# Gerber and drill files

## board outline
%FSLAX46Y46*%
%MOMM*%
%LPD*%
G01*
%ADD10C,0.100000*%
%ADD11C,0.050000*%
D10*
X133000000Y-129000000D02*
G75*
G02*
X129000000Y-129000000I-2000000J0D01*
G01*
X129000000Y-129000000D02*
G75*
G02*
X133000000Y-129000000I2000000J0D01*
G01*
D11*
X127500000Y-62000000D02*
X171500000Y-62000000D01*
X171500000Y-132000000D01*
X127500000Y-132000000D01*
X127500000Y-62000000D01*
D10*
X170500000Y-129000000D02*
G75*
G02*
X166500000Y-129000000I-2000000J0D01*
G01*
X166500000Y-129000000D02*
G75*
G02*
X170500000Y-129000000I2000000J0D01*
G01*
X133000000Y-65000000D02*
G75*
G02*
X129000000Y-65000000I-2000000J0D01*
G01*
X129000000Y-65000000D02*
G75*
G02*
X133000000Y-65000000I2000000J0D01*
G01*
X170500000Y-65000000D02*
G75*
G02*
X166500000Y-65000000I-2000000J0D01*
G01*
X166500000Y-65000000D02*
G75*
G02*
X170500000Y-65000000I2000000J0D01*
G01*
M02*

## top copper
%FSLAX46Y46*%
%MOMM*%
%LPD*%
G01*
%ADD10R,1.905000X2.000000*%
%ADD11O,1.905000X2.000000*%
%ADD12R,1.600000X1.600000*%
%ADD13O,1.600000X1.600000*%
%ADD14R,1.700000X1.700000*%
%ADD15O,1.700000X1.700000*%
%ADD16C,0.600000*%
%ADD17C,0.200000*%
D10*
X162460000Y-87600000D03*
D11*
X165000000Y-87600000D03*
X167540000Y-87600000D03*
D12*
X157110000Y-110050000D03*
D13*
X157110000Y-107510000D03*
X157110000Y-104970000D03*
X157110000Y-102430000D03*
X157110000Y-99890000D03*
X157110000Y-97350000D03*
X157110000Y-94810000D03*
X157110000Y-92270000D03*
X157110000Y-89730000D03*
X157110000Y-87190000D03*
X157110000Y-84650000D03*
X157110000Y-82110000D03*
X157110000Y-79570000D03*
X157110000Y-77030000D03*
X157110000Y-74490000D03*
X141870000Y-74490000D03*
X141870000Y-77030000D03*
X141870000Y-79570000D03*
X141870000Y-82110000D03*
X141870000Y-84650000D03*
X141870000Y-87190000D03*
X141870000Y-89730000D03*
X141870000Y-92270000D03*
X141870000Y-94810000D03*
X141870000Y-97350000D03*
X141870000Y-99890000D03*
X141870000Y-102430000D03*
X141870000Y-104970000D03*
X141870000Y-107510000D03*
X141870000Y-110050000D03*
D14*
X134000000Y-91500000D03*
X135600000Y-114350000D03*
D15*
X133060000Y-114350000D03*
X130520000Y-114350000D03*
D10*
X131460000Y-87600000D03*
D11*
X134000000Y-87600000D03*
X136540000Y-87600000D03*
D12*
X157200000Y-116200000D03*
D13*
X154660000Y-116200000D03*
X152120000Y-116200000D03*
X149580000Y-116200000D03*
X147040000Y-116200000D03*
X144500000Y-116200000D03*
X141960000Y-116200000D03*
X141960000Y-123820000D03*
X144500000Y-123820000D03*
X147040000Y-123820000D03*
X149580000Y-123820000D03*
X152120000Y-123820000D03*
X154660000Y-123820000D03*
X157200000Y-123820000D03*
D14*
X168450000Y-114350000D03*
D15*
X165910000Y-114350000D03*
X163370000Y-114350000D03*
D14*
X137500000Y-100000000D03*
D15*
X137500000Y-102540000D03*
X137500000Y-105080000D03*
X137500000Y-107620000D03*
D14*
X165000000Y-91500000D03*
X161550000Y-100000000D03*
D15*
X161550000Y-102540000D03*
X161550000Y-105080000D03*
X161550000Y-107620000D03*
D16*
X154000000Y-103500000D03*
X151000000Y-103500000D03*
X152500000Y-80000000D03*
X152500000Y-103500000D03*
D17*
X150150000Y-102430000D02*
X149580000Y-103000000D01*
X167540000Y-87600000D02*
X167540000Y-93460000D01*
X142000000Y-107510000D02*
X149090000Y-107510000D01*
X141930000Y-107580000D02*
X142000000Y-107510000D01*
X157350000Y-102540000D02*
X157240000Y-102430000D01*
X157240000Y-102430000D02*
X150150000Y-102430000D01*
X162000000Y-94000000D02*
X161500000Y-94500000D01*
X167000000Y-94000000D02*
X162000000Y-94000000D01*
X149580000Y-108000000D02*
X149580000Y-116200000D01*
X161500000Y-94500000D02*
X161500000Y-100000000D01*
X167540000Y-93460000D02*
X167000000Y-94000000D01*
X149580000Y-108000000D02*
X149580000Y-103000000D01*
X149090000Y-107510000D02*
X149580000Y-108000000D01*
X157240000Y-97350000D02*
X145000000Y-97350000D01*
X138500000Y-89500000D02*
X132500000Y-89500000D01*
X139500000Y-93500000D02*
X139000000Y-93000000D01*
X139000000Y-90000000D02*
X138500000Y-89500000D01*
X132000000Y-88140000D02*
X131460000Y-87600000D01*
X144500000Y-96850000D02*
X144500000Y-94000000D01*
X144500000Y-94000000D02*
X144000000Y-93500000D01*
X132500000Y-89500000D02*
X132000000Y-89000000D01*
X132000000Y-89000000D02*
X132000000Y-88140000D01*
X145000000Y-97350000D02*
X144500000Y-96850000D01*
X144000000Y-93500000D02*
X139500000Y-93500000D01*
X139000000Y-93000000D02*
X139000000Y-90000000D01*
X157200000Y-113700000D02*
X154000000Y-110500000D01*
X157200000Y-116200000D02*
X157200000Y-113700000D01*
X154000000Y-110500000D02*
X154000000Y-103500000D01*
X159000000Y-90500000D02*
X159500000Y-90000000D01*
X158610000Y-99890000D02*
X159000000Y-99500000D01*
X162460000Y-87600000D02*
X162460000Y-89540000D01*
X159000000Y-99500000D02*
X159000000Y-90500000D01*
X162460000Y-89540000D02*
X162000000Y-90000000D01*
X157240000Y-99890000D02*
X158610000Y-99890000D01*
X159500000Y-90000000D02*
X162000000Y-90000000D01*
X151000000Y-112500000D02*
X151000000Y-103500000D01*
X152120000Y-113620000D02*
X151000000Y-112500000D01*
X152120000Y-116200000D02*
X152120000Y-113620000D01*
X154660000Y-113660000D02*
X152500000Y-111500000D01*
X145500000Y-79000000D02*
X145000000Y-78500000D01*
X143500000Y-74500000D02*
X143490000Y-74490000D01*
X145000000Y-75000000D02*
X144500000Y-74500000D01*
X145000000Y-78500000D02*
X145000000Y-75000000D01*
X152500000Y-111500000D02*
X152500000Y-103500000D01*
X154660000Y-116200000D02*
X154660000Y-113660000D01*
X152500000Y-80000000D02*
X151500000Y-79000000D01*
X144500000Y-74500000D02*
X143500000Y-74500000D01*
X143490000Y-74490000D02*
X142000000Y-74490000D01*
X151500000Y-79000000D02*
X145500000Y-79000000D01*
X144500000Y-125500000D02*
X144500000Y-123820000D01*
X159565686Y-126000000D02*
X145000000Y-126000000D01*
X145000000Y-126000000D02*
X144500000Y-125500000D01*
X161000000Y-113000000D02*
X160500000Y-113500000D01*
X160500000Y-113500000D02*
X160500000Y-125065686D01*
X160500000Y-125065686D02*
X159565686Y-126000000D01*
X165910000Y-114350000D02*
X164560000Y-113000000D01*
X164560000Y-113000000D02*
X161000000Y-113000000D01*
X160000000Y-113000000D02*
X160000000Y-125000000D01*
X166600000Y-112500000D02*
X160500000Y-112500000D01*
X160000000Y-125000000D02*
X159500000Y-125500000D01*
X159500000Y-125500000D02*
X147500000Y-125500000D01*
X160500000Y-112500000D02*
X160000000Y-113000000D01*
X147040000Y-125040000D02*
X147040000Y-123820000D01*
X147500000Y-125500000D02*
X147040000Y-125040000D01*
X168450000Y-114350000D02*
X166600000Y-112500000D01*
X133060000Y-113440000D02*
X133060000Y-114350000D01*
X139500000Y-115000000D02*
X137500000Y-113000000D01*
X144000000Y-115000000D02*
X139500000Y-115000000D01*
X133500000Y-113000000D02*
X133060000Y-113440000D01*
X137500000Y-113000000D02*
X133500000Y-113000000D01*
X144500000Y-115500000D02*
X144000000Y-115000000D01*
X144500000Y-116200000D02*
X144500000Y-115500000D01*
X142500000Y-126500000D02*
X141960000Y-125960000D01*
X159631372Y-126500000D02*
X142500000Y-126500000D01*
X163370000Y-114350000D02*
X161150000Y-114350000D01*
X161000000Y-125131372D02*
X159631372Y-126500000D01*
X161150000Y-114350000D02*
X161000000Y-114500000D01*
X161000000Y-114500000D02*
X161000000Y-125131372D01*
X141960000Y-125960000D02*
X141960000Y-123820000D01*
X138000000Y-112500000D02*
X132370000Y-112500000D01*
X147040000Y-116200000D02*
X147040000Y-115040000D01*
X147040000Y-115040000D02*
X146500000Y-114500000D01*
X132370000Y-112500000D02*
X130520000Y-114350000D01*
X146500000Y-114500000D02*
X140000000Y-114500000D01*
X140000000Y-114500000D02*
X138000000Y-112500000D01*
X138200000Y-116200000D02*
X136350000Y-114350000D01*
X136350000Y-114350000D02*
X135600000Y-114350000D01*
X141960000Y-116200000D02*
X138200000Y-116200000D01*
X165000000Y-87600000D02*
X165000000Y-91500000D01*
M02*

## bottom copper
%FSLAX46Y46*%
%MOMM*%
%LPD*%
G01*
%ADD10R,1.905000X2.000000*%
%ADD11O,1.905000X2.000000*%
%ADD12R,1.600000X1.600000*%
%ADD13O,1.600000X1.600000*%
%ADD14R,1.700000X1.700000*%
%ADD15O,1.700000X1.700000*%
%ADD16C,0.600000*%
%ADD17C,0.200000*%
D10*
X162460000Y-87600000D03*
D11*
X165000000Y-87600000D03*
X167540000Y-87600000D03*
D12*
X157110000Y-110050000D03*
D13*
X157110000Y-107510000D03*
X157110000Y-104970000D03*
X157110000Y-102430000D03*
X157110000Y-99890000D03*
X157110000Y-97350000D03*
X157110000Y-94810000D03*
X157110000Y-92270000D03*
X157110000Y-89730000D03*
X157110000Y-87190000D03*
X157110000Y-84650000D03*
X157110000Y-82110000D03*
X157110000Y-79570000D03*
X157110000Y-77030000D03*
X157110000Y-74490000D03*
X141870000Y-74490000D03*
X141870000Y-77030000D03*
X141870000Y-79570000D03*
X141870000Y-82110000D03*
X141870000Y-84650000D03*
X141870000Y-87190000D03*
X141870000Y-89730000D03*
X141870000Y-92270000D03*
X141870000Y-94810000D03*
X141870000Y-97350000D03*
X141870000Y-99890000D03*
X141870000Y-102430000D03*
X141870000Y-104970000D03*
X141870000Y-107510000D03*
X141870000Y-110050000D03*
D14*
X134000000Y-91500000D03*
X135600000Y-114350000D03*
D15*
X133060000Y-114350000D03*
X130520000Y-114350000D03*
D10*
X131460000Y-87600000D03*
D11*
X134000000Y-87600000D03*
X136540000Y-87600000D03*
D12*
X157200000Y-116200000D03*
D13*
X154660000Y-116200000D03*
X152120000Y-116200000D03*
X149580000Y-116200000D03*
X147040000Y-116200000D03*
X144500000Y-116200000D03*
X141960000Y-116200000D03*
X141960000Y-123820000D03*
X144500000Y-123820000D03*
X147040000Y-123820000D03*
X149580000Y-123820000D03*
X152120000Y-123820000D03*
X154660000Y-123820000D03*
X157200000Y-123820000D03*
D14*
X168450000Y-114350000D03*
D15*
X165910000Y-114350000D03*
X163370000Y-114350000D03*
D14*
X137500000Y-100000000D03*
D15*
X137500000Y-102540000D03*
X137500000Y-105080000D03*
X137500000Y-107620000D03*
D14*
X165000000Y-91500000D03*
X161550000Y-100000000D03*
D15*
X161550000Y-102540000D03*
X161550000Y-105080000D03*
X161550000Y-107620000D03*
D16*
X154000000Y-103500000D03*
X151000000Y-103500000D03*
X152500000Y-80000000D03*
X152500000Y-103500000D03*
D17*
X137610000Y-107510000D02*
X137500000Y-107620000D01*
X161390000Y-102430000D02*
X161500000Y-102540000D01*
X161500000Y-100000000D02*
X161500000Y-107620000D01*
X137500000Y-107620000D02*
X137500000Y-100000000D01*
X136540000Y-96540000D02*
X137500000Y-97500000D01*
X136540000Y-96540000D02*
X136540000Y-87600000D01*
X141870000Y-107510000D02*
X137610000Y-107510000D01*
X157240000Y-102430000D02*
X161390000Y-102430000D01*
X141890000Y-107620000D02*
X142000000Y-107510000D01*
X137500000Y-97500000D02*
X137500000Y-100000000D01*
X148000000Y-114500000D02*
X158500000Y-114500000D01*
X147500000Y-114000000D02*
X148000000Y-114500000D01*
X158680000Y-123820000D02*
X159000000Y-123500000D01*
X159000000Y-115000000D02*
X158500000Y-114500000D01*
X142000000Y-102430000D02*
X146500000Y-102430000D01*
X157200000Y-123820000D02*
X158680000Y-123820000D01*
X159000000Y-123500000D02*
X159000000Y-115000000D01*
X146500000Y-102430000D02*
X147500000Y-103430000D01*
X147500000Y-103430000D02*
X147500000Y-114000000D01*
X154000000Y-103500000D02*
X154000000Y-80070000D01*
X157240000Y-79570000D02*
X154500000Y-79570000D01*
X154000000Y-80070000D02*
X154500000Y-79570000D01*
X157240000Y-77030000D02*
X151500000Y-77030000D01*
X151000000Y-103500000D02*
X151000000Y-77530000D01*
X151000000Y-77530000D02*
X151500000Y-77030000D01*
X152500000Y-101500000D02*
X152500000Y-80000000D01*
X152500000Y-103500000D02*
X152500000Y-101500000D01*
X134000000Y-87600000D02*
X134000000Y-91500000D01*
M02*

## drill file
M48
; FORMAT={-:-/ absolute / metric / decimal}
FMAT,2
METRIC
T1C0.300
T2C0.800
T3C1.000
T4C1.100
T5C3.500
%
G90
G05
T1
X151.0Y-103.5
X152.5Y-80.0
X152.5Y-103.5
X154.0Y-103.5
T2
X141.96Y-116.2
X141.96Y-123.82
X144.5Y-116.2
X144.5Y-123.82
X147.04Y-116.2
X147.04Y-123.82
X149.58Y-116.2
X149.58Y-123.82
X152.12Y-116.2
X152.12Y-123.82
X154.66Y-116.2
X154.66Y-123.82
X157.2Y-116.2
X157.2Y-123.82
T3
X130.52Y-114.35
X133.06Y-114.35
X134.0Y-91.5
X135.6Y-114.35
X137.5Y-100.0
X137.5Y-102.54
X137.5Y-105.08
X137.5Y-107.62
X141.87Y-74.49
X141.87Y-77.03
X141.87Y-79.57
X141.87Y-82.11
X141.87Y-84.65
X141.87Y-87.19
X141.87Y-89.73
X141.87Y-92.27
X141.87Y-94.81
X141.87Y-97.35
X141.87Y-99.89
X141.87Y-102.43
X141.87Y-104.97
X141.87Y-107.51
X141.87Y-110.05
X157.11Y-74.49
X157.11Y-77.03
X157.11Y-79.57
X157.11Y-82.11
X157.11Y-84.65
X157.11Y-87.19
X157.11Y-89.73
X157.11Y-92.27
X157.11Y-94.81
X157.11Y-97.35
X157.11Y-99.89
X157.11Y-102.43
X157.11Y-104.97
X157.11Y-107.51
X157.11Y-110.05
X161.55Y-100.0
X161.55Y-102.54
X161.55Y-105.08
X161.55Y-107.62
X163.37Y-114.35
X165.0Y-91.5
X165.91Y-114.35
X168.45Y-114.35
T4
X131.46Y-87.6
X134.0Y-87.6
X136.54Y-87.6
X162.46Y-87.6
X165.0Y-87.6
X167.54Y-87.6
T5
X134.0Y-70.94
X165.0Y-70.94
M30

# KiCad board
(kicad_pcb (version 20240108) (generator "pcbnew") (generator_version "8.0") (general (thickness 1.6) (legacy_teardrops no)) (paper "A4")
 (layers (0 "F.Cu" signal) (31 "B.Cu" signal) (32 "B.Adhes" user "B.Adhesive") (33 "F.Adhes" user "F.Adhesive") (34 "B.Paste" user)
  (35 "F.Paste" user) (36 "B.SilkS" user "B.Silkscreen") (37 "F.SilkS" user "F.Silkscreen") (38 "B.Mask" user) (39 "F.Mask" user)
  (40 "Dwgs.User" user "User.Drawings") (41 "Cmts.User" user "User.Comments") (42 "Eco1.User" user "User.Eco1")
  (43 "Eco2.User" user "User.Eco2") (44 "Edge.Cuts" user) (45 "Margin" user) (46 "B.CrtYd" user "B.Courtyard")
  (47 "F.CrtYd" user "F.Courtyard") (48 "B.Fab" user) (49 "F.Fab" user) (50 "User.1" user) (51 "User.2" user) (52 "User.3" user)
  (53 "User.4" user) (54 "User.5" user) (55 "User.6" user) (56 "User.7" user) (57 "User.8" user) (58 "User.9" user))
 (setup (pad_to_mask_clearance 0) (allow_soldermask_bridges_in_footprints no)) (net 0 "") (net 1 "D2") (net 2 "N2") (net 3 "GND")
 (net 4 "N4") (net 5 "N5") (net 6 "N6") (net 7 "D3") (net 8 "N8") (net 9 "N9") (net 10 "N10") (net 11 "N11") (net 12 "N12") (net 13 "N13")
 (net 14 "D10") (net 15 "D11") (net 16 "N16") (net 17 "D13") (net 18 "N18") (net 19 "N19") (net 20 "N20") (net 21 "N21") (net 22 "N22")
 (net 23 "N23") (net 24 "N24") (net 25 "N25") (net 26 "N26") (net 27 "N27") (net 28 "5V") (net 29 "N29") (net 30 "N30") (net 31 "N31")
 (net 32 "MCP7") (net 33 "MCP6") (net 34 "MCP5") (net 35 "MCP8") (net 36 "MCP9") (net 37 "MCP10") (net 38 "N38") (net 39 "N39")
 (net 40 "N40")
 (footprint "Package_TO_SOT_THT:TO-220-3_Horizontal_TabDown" (layer "F.Cu") (at 162.46 87.6)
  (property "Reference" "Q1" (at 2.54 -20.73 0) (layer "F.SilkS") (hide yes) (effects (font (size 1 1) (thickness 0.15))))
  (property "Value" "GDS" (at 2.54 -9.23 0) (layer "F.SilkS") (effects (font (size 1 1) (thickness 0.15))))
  (pad "" np_thru_hole oval (at 2.54 -16.66) (size 3.5 3.5) (drill 3.5) (layers "*.Cu" "*.Mask"))
  (pad "1" thru_hole rect (at 0 0) (size 1.905 2) (drill 1.1) (layers "*.Cu" "*.Mask") (remove_unused_layers no) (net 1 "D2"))
  (pad "2" thru_hole oval (at 2.54 0) (size 1.905 2) (drill 1.1) (layers "*.Cu" "*.Mask") (remove_unused_layers no) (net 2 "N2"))
  (pad "3" thru_hole oval (at 5.08 0) (size 1.905 2) (drill 1.1) (layers "*.Cu" "*.Mask") (remove_unused_layers no) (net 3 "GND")))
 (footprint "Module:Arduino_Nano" (layer "F.Cu") (at 157.11 110.05 180)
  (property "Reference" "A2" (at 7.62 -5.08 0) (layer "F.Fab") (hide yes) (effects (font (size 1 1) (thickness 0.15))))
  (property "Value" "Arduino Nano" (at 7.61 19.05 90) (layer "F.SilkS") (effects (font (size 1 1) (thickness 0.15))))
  (pad "1" thru_hole rect (at 0 0 180) (size 1.6 1.6) (drill 1) (layers "*.Cu" "*.Mask") (remove_unused_layers no) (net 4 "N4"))
  (pad "2" thru_hole oval (at 0 2.54 180) (size 1.6 1.6) (drill 1) (layers "*.Cu" "*.Mask") (remove_unused_layers no) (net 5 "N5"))
  (pad "3" thru_hole oval (at 0 5.08 180) (size 1.6 1.6) (drill 1) (layers "*.Cu" "*.Mask") (remove_unused_layers no) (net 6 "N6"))
  (pad "4" thru_hole oval (at 0 7.62 180) (size 1.6 1.6) (drill 1) (layers "*.Cu" "*.Mask") (remove_unused_layers no) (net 3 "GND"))
  (pad "5" thru_hole oval (at 0 10.16 180) (size 1.6 1.6) (drill 1) (layers "*.Cu" "*.Mask") (remove_unused_layers no) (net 1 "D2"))
  (pad "6" thru_hole oval (at 0 12.7 180) (size 1.6 1.6) (drill 1) (layers "*.Cu" "*.Mask") (remove_unused_layers no) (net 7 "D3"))
  (pad "7" thru_hole oval (at 0 15.24 180) (size 1.6 1.6) (drill 1) (layers "*.Cu" "*.Mask") (remove_unused_layers no) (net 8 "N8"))
  (pad "8" thru_hole oval (at 0 17.78 180) (size 1.6 1.6) (drill 1) (layers "*.Cu" "*.Mask") (remove_unused_layers no) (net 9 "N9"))
  (pad "9" thru_hole oval (at 0 20.32 180) (size 1.6 1.6) (drill 1) (layers "*.Cu" "*.Mask") (remove_unused_layers no) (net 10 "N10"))
  (pad "10" thru_hole oval (at 0 22.86 180) (size 1.6 1.6) (drill 1) (layers "*.Cu" "*.Mask") (remove_unused_layers no) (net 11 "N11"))
  (pad "11" thru_hole oval (at 0 25.4 180) (size 1.6 1.6) (drill 1) (layers "*.Cu" "*.Mask") (remove_unused_layers no) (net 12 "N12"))
  (pad "12" thru_hole oval (at 0 27.94 180) (size 1.6 1.6) (drill 1) (layers "*.Cu" "*.Mask") (remove_unused_layers no) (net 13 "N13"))
  (pad "13" thru_hole oval (at 0 30.48 180) (size 1.6 1.6) (drill 1) (layers "*.Cu" "*.Mask") (remove_unused_layers no) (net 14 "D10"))
  (pad "14" thru_hole oval (at 0 33.02 180) (size 1.6 1.6) (drill 1) (layers "*.Cu" "*.Mask") (remove_unused_layers no) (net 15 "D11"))
  (pad "15" thru_hole oval (at 0 35.56 180) (size 1.6 1.6) (drill 1) (layers "*.Cu" "*.Mask") (remove_unused_layers no) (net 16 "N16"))
  (pad "16" thru_hole oval (at 15.24 35.56 180) (size 1.6 1.6) (drill 1) (layers "*.Cu" "*.Mask") (remove_unused_layers no) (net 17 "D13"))
  (pad "17" thru_hole oval (at 15.24 33.02 180) (size 1.6 1.6) (drill 1) (layers "*.Cu" "*.Mask") (remove_unused_layers no) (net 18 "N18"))
  (pad "18" thru_hole oval (at 15.24 30.48 180) (size 1.6 1.6) (drill 1) (layers "*.Cu" "*.Mask") (remove_unused_layers no) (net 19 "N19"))
  (pad "19" thru_hole oval (at 15.24 27.94 180) (size 1.6 1.6) (drill 1) (layers "*.Cu" "*.Mask") (remove_unused_layers no) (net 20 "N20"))
  (pad "20" thru_hole oval (at 15.24 25.4 180) (size 1.6 1.6) (drill 1) (layers "*.Cu" "*.Mask") (remove_unused_layers no) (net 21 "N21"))
  (pad "21" thru_hole oval (at 15.24 22.86 180) (size 1.6 1.6) (drill 1) (layers "*.Cu" "*.Mask") (remove_unused_layers no) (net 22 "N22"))
  (pad "22" thru_hole oval (at 15.24 20.32 180) (size 1.6 1.6) (drill 1) (layers "*.Cu" "*.Mask") (remove_unused_layers no) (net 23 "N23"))
  (pad "23" thru_hole oval (at 15.24 17.78 180) (size 1.6 1.6) (drill 1) (layers "*.Cu" "*.Mask") (remove_unused_layers no) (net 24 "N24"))
  (pad "24" thru_hole oval (at 15.24 15.24 180) (size 1.6 1.6) (drill 1) (layers "*.Cu" "*.Mask") (remove_unused_layers no) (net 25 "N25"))
  (pad "25" thru_hole oval (at 15.24 12.7 180) (size 1.6 1.6) (drill 1) (layers "*.Cu" "*.Mask") (remove_unused_layers no) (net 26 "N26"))
  (pad "26" thru_hole oval (at 15.24 10.16 180) (size 1.6 1.6) (drill 1) (layers "*.Cu" "*.Mask") (remove_unused_layers no) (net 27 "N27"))
  (pad "27" thru_hole oval (at 15.24 7.62 180) (size 1.6 1.6) (drill 1) (layers "*.Cu" "*.Mask") (remove_unused_layers no) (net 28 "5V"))
  (pad "28" thru_hole oval (at 15.24 5.08 180) (size 1.6 1.6) (drill 1) (layers "*.Cu" "*.Mask") (remove_unused_layers no) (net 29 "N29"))
  (pad "29" thru_hole oval (at 15.24 2.54 180) (size 1.6 1.6) (drill 1) (layers "*.Cu" "*.Mask") (remove_unused_layers no) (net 3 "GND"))
  (pad "30" thru_hole oval (at 15.24 0 180) (size 1.6 1.6) (drill 1) (layers "*.Cu" "*.Mask") (remove_unused_layers no) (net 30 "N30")))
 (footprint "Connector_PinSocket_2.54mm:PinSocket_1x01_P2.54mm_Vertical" (layer "F.Cu") (at 134 91.5)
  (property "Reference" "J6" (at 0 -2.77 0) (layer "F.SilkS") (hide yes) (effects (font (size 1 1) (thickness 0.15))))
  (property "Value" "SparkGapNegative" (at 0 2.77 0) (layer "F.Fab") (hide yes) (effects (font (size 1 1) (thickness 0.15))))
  (pad "1" thru_hole rect (at 0 0) (size 1.7 1.7) (drill 1) (layers "*.Cu" "*.Mask") (remove_unused_layers no) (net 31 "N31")))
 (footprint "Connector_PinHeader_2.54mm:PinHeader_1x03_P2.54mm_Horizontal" (layer "F.Cu") (at 135.6 114.35 -90)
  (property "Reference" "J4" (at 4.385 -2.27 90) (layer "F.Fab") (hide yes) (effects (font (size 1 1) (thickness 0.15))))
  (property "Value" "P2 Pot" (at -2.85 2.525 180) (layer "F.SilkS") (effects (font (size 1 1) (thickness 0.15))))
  (pad "1" thru_hole rect (at 0 0 270) (size 1.7 1.7) (drill 1) (layers "*.Cu" "*.Mask") (remove_unused_layers no) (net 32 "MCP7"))
  (pad "2" thru_hole oval (at 0 2.54 270) (size 1.7 1.7) (drill 1) (layers "*.Cu" "*.Mask") (remove_unused_layers no) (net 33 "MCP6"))
  (pad "3" thru_hole oval (at 0 5.08 270) (size 1.7 1.7) (drill 1) (layers "*.Cu" "*.Mask") (remove_unused_layers no) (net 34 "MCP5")))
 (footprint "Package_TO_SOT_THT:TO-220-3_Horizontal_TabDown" (layer "F.Cu") (at 131.46 87.6)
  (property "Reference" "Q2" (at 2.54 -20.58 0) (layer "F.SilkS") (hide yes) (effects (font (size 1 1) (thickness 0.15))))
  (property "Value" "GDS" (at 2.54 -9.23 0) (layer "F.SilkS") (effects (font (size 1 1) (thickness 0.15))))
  (pad "" np_thru_hole oval (at 2.54 -16.66) (size 3.5 3.5) (drill 3.5) (layers "*.Cu" "*.Mask"))
  (pad "1" thru_hole rect (at 0 0) (size 1.905 2) (drill 1.1) (layers "*.Cu" "*.Mask") (remove_unused_layers no) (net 7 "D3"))
  (pad "2" thru_hole oval (at 2.54 0) (size 1.905 2) (drill 1.1) (layers "*.Cu" "*.Mask") (remove_unused_layers no) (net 31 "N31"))
  (pad "3" thru_hole oval (at 5.08 0) (size 1.905 2) (drill 1.1) (layers "*.Cu" "*.Mask") (remove_unused_layers no) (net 3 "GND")))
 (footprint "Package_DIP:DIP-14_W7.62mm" (layer "F.Cu") (at 157.2 116.2 -90)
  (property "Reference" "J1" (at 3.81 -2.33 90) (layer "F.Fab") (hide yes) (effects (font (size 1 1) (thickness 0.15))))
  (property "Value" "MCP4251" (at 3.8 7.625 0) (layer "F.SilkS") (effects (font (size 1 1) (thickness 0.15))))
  (pad "1" thru_hole rect (at 0 0 270) (size 1.6 1.6) (drill 0.8) (layers "*.Cu" "*.Mask") (remove_unused_layers no) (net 14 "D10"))
  (pad "2" thru_hole oval (at 0 2.54 270) (size 1.6 1.6) (drill 0.8) (layers "*.Cu" "*.Mask") (remove_unused_layers no) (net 17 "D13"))
  (pad "3" thru_hole oval (at 0 5.08 270) (size 1.6 1.6) (drill 0.8) (layers "*.Cu" "*.Mask") (remove_unused_layers no) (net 15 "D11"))
  (pad "4" thru_hole oval (at 0 7.62 270) (size 1.6 1.6) (drill 0.8) (layers "*.Cu" "*.Mask") (remove_unused_layers no) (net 3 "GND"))
  (pad "5" thru_hole oval (at 0 10.16 270) (size 1.6 1.6) (drill 0.8) (layers "*.Cu" "*.Mask") (remove_unused_layers no) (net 34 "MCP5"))
  (pad "6" thru_hole oval (at 0 12.7 270) (size 1.6 1.6) (drill 0.8) (layers "*.Cu" "*.Mask") (remove_unused_layers no) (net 33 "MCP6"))
  (pad "7" thru_hole oval (at 0 15.24 270) (size 1.6 1.6) (drill 0.8) (layers "*.Cu" "*.Mask") (remove_unused_layers no) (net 32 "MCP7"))
  (pad "8" thru_hole oval (at 7.62 15.24 270) (size 1.6 1.6) (drill 0.8) (layers "*.Cu" "*.Mask") (remove_unused_layers no) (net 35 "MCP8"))
  (pad "9" thru_hole oval (at 7.62 12.7 270) (size 1.6 1.6) (drill 0.8) (layers "*.Cu" "*.Mask") (remove_unused_layers no) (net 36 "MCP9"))
  (pad "10" thru_hole oval (at 7.62 10.16 270) (size 1.6 1.6) (drill 0.8) (layers "*.Cu" "*.Mask") (remove_unused_layers no)
   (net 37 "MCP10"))
  (pad "11" thru_hole oval (at 7.62 7.62 270) (size 1.6 1.6) (drill 0.8) (layers "*.Cu" "*.Mask") (remove_unused_layers no) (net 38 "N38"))
  (pad "12" thru_hole oval (at 7.62 5.08 270) (size 1.6 1.6) (drill 0.8) (layers "*.Cu" "*.Mask") (remove_unused_layers no) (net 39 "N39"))
  (pad "13" thru_hole oval (at 7.62 2.54 270) (size 1.6 1.6) (drill 0.8) (layers "*.Cu" "*.Mask") (remove_unused_layers no) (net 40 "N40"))
  (pad "14" thru_hole oval (at 7.62 0 270) (size 1.6 1.6) (drill 0.8) (layers "*.Cu" "*.Mask") (remove_unused_layers no) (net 28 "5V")))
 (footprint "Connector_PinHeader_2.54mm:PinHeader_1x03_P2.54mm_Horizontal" (layer "F.Cu") (at 168.45 114.35 -90)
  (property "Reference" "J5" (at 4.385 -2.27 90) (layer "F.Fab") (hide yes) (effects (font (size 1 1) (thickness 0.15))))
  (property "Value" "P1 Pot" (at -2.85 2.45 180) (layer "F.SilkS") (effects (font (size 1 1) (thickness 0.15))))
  (pad "1" thru_hole rect (at 0 0 270) (size 1.7 1.7) (drill 1) (layers "*.Cu" "*.Mask") (remove_unused_layers no) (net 37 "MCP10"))
  (pad "2" thru_hole oval (at 0 2.54 270) (size 1.7 1.7) (drill 1) (layers "*.Cu" "*.Mask") (remove_unused_layers no) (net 36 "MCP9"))
  (pad "3" thru_hole oval (at 0 5.08 270) (size 1.7 1.7) (drill 1) (layers "*.Cu" "*.Mask") (remove_unused_layers no) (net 35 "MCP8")))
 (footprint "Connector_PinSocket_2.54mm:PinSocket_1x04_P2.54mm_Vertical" (layer "F.Cu") (at 137.5 100)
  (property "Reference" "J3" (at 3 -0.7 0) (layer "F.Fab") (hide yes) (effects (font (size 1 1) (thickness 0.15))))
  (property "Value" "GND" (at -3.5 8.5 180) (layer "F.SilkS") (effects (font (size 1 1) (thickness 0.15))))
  (pad "1" thru_hole rect (at 0 0) (size 1.7 1.7) (drill 1) (layers "*.Cu" "*.Mask") (remove_unused_layers no) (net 3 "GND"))
  (pad "2" thru_hole oval (at 0 2.54) (size 1.7 1.7) (drill 1) (layers "*.Cu" "*.Mask") (remove_unused_layers no) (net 3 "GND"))
  (pad "3" thru_hole oval (at 0 5.08) (size 1.7 1.7) (drill 1) (layers "*.Cu" "*.Mask") (remove_unused_layers no) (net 3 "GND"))
  (pad "4" thru_hole oval (at 0 7.62) (size 1.7 1.7) (drill 1) (layers "*.Cu" "*.Mask") (remove_unused_layers no) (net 3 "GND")))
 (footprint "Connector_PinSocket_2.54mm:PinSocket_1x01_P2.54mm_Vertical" (layer "F.Cu") (at 165 91.5)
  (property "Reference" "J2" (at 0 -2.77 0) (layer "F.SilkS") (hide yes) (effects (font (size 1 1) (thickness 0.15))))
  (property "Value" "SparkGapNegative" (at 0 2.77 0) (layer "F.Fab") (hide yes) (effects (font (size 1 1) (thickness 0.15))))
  (pad "1" thru_hole rect (at 0 0) (size 1.7 1.7) (drill 1) (layers "*.Cu" "*.Mask") (remove_unused_layers no) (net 2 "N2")))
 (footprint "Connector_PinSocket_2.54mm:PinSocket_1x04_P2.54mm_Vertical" (layer "F.Cu") (at 161.55 100)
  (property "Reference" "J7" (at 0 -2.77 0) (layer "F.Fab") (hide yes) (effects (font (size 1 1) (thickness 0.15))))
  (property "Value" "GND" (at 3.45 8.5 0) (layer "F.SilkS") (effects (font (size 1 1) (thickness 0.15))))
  (pad "1" thru_hole rect (at 0 0) (size 1.7 1.7) (drill 1) (layers "*.Cu" "*.Mask") (remove_unused_layers no) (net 3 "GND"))
  (pad "2" thru_hole oval (at 0 2.54) (size 1.7 1.7) (drill 1) (layers "*.Cu" "*.Mask") (remove_unused_layers no) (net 3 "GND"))
  (pad "3" thru_hole oval (at 0 5.08) (size 1.7 1.7) (drill 1) (layers "*.Cu" "*.Mask") (remove_unused_layers no) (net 3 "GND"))
  (pad "4" thru_hole oval (at 0 7.62) (size 1.7 1.7) (drill 1) (layers "*.Cu" "*.Mask") (remove_unused_layers no) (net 3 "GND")))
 (gr_circle (center 131 129) (end 133 129) (stroke (width 0.1) (type default)) (fill none) (layer "Edge.Cuts"))
 (gr_rect (start 127.5 62) (end 171.5 132) (stroke (width 0.05) (type default)) (fill none) (layer "Edge.Cuts"))
 (gr_circle (center 168.5 129) (end 170.5 129) (stroke (width 0.1) (type default)) (fill none) (layer "Edge.Cuts"))
 (gr_circle (center 131 65) (end 133 65) (stroke (width 0.1) (type default)) (fill none) (layer "Edge.Cuts"))
 (gr_circle (center 168.5 65) (end 170.5 65) (stroke (width 0.1) (type default)) (fill none) (layer "Edge.Cuts"))
 (segment (start 150.15 102.43) (end 149.58 103) (width 0.2) (layer "F.Cu") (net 3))
 (segment (start 167.54 87.6) (end 167.54 93.46) (width 0.2) (layer "F.Cu") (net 3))
 (segment (start 142 107.51) (end 149.09 107.51) (width 0.2) (layer "F.Cu") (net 3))
 (segment (start 141.93 107.58) (end 142 107.51) (width 0.2) (layer "F.Cu") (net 3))
 (segment (start 157.35 102.54) (end 157.24 102.43) (width 0.2) (layer "F.Cu") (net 3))
 (segment (start 157.24 102.43) (end 150.15 102.43) (width 0.2) (layer "F.Cu") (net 3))
 (segment (start 162 94) (end 161.5 94.5) (width 0.2) (layer "F.Cu") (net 3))
 (segment (start 167 94) (end 162 94) (width 0.2) (layer "F.Cu") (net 3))
 (segment (start 149.58 108) (end 149.58 116.2) (width 0.2) (layer "F.Cu") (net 3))
 (segment (start 161.5 94.5) (end 161.5 100) (width 0.2) (layer "F.Cu") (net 3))
 (segment (start 167.54 93.46) (end 167 94) (width 0.2) (layer "F.Cu") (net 3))
 (segment (start 149.58 108) (end 149.58 103) (width 0.2) (layer "F.Cu") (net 3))
 (segment (start 149.09 107.51) (end 149.58 108) (width 0.2) (layer "F.Cu") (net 3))
 (segment (start 137.61 107.51) (end 137.5 107.62) (width 0.2) (layer "B.Cu") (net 3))
 (segment (start 161.39 102.43) (end 161.5 102.54) (width 0.2) (layer "B.Cu") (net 3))
 (segment (start 161.5 100) (end 161.5 107.62) (width 0.2) (layer "B.Cu") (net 3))
 (segment (start 137.5 107.62) (end 137.5 100) (width 0.2) (layer "B.Cu") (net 3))
 (segment (start 136.54 96.54) (end 137.5 97.5) (width 0.2) (layer "B.Cu") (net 3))
 (segment (start 136.54 96.54) (end 136.54 87.6) (width 0.2) (layer "B.Cu") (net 3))
 (segment (start 141.87 107.51) (end 137.61 107.51) (width 0.2) (layer "B.Cu") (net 3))
 (segment (start 157.24 102.43) (end 161.39 102.43) (width 0.2) (layer "B.Cu") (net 3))
 (segment (start 141.89 107.62) (end 142 107.51) (width 0.2) (layer "B.Cu") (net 3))
 (segment (start 137.5 97.5) (end 137.5 100) (width 0.2) (layer "B.Cu") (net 3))
 (segment (start 157.24 97.35) (end 145 97.35) (width 0.2) (layer "F.Cu") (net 7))
 (segment (start 138.5 89.5) (end 132.5 89.5) (width 0.2) (layer "F.Cu") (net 7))
 (segment (start 139.5 93.5) (end 139 93) (width 0.2) (layer "F.Cu") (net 7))
 (segment (start 139 90) (end 138.5 89.5) (width 0.2) (layer "F.Cu") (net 7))
 (segment (start 132 88.14) (end 131.46 87.6) (width 0.2) (layer "F.Cu") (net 7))
 (segment (start 144.5 96.85) (end 144.5 94) (width 0.2) (layer "F.Cu") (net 7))
 (segment (start 144.5 94) (end 144 93.5) (width 0.2) (layer "F.Cu") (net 7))
 (segment (start 132.5 89.5) (end 132 89) (width 0.2) (layer "F.Cu") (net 7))
 (segment (start 132 89) (end 132 88.14) (width 0.2) (layer "F.Cu") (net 7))
 (segment (start 145 97.35) (end 144.5 96.85) (width 0.2) (layer "F.Cu") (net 7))
 (segment (start 144 93.5) (end 139.5 93.5) (width 0.2) (layer "F.Cu") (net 7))
 (segment (start 139 93) (end 139 90) (width 0.2) (layer "F.Cu") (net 7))
 (segment (start 148 114.5) (end 158.5 114.5) (width 0.2) (layer "B.Cu") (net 28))
 (segment (start 147.5 114) (end 148 114.5) (width 0.2) (layer "B.Cu") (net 28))
 (segment (start 158.68 123.82) (end 159 123.5) (width 0.2) (layer "B.Cu") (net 28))
 (segment (start 159 115) (end 158.5 114.5) (width 0.2) (layer "B.Cu") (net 28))
 (segment (start 142 102.43) (end 146.5 102.43) (width 0.2) (layer "B.Cu") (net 28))
 (segment (start 157.2 123.82) (end 158.68 123.82) (width 0.2) (layer "B.Cu") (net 28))
 (segment (start 159 123.5) (end 159 115) (width 0.2) (layer "B.Cu") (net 28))
 (segment (start 146.5 102.43) (end 147.5 103.43) (width 0.2) (layer "B.Cu") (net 28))
 (segment (start 147.5 103.43) (end 147.5 114) (width 0.2) (layer "B.Cu") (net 28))
 (segment (start 157.2 113.7) (end 154 110.5) (width 0.2) (layer "F.Cu") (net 14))
 (segment (start 157.2 116.2) (end 157.2 113.7) (width 0.2) (layer "F.Cu") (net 14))
 (segment (start 154 110.5) (end 154 103.5) (width 0.2) (layer "F.Cu") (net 14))
 (via (at 154 103.5) (size 0.6) (drill 0.3) (layers "F.Cu" "B.Cu") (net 14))
 (segment (start 154 103.5) (end 154 80.07) (width 0.2) (layer "B.Cu") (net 14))
 (segment (start 157.24 79.57) (end 154.5 79.57) (width 0.2) (layer "B.Cu") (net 14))
 (segment (start 154 80.07) (end 154.5 79.57) (width 0.2) (layer "B.Cu") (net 14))
 (segment (start 159 90.5) (end 159.5 90) (width 0.2) (layer "F.Cu") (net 1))
 (segment (start 158.61 99.89) (end 159 99.5) (width 0.2) (layer "F.Cu") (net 1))
 (segment (start 162.46 87.6) (end 162.46 89.54) (width 0.2) (layer "F.Cu") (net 1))
 (segment (start 159 99.5) (end 159 90.5) (width 0.2) (layer "F.Cu") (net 1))
 (segment (start 162.46 89.54) (end 162 90) (width 0.2) (layer "F.Cu") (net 1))
 (segment (start 157.24 99.89) (end 158.61 99.89) (width 0.2) (layer "F.Cu") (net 1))
 (segment (start 159.5 90) (end 162 90) (width 0.2) (layer "F.Cu") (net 1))
 (segment (start 151 112.5) (end 151 103.5) (width 0.2) (layer "F.Cu") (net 15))
 (segment (start 152.12 113.62) (end 151 112.5) (width 0.2) (layer "F.Cu") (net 15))
 (segment (start 152.12 116.2) (end 152.12 113.62) (width 0.2) (layer "F.Cu") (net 15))
 (via (at 151 103.5) (size 0.6) (drill 0.3) (layers "F.Cu" "B.Cu") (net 15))
 (segment (start 157.24 77.03) (end 151.5 77.03) (width 0.2) (layer "B.Cu") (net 15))
 (segment (start 151 103.5) (end 151 77.53) (width 0.2) (layer "B.Cu") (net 15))
 (segment (start 151 77.53) (end 151.5 77.03) (width 0.2) (layer "B.Cu") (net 15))
 (segment (start 154.66 113.66) (end 152.5 111.5) (width 0.2) (layer "F.Cu") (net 17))
 (segment (start 145.5 79) (end 145 78.5) (width 0.2) (layer "F.Cu") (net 17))
 (segment (start 143.5 74.5) (end 143.49 74.49) (width 0.2) (layer "F.Cu") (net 17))
 (segment (start 145 75) (end 144.5 74.5) (width 0.2) (layer "F.Cu") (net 17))
 (segment (start 145 78.5) (end 145 75) (width 0.2) (layer "F.Cu") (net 17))
 (segment (start 152.5 111.5) (end 152.5 103.5) (width 0.2) (layer "F.Cu") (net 17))
 (segment (start 154.66 116.2) (end 154.66 113.66) (width 0.2) (layer "F.Cu") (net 17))
 (segment (start 152.5 80) (end 151.5 79) (width 0.2) (layer "F.Cu") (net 17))
 (segment (start 144.5 74.5) (end 143.5 74.5) (width 0.2) (layer "F.Cu") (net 17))
 (segment (start 143.49 74.49) (end 142 74.49) (width 0.2) (layer "F.Cu") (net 17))
 (segment (start 151.5 79) (end 145.5 79) (width 0.2) (layer "F.Cu") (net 17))
 (via (at 152.5 80) (size 0.6) (drill 0.3) (layers "F.Cu" "B.Cu") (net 17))
 (via (at 152.5 103.5) (size 0.6) (drill 0.3) (layers "F.Cu" "B.Cu") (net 17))
 (segment (start 152.5 101.5) (end 152.5 80) (width 0.2) (layer "B.Cu") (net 17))
 (segment (start 152.5 103.5) (end 152.5 101.5) (width 0.2) (layer "B.Cu") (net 17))
 (segment (start 144.5 125.5) (end 144.5 123.82) (width 0.2) (layer "F.Cu") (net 36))
 (segment (start 159.565686 126) (end 145 126) (width 0.2) (layer "F.Cu") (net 36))
 (segment (start 145 126) (end 144.5 125.5) (width 0.2) (layer "F.Cu") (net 36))
 (segment (start 161 113) (end 160.5 113.5) (width 0.2) (layer "F.Cu") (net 36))
 (segment (start 160.5 113.5) (end 160.5 125.065686) (width 0.2) (layer "F.Cu") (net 36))
 (segment (start 160.5 125.065686) (end 159.565686 126) (width 0.2) (layer "F.Cu") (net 36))
 (segment (start 165.91 114.35) (end 164.56 113) (width 0.2) (layer "F.Cu") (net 36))
 (segment (start 164.56 113) (end 161 113) (width 0.2) (layer "F.Cu") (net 36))
 (segment (start 160 113) (end 160 125) (width 0.2) (layer "F.Cu") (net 37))
 (segment (start 166.6 112.5) (end 160.5 112.5) (width 0.2) (layer "F.Cu") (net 37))
 (segment (start 160 125) (end 159.5 125.5) (width 0.2) (layer "F.Cu") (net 37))
 (segment (start 159.5 125.5) (end 147.5 125.5) (width 0.2) (layer "F.Cu") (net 37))
 (segment (start 160.5 112.5) (end 160 113) (width 0.2) (layer "F.Cu") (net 37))
 (segment (start 147.04 125.04) (end 147.04 123.82) (width 0.2) (layer "F.Cu") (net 37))
 (segment (start 147.5 125.5) (end 147.04 125.04) (width 0.2) (layer "F.Cu") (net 37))
 (segment (start 168.45 114.35) (end 166.6 112.5) (width 0.2) (layer "F.Cu") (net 37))
 (segment (start 133.06 113.44) (end 133.06 114.35) (width 0.2) (layer "F.Cu") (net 33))
 (segment (start 139.5 115) (end 137.5 113) (width 0.2) (layer "F.Cu") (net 33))
 (segment (start 144 115) (end 139.5 115) (width 0.2) (layer "F.Cu") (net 33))
 (segment (start 133.5 113) (end 133.06 113.44) (width 0.2) (layer "F.Cu") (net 33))
 (segment (start 137.5 113) (end 133.5 113) (width 0.2) (layer "F.Cu") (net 33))
 (segment (start 144.5 115.5) (end 144 115) (width 0.2) (layer "F.Cu") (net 33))
 (segment (start 144.5 116.2) (end 144.5 115.5) (width 0.2) (layer "F.Cu") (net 33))
 (segment (start 142.5 126.5) (end 141.96 125.96) (width 0.2) (layer "F.Cu") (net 35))
 (segment (start 159.631372 126.5) (end 142.5 126.5) (width 0.2) (layer "F.Cu") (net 35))
 (segment (start 163.37 114.35) (end 161.15 114.35) (width 0.2) (layer "F.Cu") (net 35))
 (segment (start 161 125.131372) (end 159.631372 126.5) (width 0.2) (layer "F.Cu") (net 35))
 (segment (start 161.15 114.35) (end 161 114.5) (width 0.2) (layer "F.Cu") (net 35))
 (segment (start 161 114.5) (end 161 125.131372) (width 0.2) (layer "F.Cu") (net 35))
 (segment (start 141.96 125.96) (end 141.96 123.82) (width 0.2) (layer "F.Cu") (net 35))
 (segment (start 138 112.5) (end 132.37 112.5) (width 0.2) (layer "F.Cu") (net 34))
 (segment (start 147.04 116.2) (end 147.04 115.04) (width 0.2) (layer "F.Cu") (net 34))
 (segment (start 147.04 115.04) (end 146.5 114.5) (width 0.2) (layer "F.Cu") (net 34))
 (segment (start 132.37 112.5) (end 130.52 114.35) (width 0.2) (layer "F.Cu") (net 34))
 (segment (start 146.5 114.5) (end 140 114.5) (width 0.2) (layer "F.Cu") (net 34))
 (segment (start 140 114.5) (end 138 112.5) (width 0.2) (layer "F.Cu") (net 34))
 (segment (start 138.2 116.2) (end 136.35 114.35) (width 0.2) (layer "F.Cu") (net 32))
 (segment (start 136.35 114.35) (end 135.6 114.35) (width 0.2) (layer "F.Cu") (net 32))
 (segment (start 141.96 116.2) (end 138.2 116.2) (width 0.2) (layer "F.Cu") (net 32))
 (segment (start 165 87.6) (end 165 91.5) (width 0.2) (layer "F.Cu") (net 2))
 (segment (start 134 87.6) (end 134 91.5) (width 0.2) (layer "B.Cu") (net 31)))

